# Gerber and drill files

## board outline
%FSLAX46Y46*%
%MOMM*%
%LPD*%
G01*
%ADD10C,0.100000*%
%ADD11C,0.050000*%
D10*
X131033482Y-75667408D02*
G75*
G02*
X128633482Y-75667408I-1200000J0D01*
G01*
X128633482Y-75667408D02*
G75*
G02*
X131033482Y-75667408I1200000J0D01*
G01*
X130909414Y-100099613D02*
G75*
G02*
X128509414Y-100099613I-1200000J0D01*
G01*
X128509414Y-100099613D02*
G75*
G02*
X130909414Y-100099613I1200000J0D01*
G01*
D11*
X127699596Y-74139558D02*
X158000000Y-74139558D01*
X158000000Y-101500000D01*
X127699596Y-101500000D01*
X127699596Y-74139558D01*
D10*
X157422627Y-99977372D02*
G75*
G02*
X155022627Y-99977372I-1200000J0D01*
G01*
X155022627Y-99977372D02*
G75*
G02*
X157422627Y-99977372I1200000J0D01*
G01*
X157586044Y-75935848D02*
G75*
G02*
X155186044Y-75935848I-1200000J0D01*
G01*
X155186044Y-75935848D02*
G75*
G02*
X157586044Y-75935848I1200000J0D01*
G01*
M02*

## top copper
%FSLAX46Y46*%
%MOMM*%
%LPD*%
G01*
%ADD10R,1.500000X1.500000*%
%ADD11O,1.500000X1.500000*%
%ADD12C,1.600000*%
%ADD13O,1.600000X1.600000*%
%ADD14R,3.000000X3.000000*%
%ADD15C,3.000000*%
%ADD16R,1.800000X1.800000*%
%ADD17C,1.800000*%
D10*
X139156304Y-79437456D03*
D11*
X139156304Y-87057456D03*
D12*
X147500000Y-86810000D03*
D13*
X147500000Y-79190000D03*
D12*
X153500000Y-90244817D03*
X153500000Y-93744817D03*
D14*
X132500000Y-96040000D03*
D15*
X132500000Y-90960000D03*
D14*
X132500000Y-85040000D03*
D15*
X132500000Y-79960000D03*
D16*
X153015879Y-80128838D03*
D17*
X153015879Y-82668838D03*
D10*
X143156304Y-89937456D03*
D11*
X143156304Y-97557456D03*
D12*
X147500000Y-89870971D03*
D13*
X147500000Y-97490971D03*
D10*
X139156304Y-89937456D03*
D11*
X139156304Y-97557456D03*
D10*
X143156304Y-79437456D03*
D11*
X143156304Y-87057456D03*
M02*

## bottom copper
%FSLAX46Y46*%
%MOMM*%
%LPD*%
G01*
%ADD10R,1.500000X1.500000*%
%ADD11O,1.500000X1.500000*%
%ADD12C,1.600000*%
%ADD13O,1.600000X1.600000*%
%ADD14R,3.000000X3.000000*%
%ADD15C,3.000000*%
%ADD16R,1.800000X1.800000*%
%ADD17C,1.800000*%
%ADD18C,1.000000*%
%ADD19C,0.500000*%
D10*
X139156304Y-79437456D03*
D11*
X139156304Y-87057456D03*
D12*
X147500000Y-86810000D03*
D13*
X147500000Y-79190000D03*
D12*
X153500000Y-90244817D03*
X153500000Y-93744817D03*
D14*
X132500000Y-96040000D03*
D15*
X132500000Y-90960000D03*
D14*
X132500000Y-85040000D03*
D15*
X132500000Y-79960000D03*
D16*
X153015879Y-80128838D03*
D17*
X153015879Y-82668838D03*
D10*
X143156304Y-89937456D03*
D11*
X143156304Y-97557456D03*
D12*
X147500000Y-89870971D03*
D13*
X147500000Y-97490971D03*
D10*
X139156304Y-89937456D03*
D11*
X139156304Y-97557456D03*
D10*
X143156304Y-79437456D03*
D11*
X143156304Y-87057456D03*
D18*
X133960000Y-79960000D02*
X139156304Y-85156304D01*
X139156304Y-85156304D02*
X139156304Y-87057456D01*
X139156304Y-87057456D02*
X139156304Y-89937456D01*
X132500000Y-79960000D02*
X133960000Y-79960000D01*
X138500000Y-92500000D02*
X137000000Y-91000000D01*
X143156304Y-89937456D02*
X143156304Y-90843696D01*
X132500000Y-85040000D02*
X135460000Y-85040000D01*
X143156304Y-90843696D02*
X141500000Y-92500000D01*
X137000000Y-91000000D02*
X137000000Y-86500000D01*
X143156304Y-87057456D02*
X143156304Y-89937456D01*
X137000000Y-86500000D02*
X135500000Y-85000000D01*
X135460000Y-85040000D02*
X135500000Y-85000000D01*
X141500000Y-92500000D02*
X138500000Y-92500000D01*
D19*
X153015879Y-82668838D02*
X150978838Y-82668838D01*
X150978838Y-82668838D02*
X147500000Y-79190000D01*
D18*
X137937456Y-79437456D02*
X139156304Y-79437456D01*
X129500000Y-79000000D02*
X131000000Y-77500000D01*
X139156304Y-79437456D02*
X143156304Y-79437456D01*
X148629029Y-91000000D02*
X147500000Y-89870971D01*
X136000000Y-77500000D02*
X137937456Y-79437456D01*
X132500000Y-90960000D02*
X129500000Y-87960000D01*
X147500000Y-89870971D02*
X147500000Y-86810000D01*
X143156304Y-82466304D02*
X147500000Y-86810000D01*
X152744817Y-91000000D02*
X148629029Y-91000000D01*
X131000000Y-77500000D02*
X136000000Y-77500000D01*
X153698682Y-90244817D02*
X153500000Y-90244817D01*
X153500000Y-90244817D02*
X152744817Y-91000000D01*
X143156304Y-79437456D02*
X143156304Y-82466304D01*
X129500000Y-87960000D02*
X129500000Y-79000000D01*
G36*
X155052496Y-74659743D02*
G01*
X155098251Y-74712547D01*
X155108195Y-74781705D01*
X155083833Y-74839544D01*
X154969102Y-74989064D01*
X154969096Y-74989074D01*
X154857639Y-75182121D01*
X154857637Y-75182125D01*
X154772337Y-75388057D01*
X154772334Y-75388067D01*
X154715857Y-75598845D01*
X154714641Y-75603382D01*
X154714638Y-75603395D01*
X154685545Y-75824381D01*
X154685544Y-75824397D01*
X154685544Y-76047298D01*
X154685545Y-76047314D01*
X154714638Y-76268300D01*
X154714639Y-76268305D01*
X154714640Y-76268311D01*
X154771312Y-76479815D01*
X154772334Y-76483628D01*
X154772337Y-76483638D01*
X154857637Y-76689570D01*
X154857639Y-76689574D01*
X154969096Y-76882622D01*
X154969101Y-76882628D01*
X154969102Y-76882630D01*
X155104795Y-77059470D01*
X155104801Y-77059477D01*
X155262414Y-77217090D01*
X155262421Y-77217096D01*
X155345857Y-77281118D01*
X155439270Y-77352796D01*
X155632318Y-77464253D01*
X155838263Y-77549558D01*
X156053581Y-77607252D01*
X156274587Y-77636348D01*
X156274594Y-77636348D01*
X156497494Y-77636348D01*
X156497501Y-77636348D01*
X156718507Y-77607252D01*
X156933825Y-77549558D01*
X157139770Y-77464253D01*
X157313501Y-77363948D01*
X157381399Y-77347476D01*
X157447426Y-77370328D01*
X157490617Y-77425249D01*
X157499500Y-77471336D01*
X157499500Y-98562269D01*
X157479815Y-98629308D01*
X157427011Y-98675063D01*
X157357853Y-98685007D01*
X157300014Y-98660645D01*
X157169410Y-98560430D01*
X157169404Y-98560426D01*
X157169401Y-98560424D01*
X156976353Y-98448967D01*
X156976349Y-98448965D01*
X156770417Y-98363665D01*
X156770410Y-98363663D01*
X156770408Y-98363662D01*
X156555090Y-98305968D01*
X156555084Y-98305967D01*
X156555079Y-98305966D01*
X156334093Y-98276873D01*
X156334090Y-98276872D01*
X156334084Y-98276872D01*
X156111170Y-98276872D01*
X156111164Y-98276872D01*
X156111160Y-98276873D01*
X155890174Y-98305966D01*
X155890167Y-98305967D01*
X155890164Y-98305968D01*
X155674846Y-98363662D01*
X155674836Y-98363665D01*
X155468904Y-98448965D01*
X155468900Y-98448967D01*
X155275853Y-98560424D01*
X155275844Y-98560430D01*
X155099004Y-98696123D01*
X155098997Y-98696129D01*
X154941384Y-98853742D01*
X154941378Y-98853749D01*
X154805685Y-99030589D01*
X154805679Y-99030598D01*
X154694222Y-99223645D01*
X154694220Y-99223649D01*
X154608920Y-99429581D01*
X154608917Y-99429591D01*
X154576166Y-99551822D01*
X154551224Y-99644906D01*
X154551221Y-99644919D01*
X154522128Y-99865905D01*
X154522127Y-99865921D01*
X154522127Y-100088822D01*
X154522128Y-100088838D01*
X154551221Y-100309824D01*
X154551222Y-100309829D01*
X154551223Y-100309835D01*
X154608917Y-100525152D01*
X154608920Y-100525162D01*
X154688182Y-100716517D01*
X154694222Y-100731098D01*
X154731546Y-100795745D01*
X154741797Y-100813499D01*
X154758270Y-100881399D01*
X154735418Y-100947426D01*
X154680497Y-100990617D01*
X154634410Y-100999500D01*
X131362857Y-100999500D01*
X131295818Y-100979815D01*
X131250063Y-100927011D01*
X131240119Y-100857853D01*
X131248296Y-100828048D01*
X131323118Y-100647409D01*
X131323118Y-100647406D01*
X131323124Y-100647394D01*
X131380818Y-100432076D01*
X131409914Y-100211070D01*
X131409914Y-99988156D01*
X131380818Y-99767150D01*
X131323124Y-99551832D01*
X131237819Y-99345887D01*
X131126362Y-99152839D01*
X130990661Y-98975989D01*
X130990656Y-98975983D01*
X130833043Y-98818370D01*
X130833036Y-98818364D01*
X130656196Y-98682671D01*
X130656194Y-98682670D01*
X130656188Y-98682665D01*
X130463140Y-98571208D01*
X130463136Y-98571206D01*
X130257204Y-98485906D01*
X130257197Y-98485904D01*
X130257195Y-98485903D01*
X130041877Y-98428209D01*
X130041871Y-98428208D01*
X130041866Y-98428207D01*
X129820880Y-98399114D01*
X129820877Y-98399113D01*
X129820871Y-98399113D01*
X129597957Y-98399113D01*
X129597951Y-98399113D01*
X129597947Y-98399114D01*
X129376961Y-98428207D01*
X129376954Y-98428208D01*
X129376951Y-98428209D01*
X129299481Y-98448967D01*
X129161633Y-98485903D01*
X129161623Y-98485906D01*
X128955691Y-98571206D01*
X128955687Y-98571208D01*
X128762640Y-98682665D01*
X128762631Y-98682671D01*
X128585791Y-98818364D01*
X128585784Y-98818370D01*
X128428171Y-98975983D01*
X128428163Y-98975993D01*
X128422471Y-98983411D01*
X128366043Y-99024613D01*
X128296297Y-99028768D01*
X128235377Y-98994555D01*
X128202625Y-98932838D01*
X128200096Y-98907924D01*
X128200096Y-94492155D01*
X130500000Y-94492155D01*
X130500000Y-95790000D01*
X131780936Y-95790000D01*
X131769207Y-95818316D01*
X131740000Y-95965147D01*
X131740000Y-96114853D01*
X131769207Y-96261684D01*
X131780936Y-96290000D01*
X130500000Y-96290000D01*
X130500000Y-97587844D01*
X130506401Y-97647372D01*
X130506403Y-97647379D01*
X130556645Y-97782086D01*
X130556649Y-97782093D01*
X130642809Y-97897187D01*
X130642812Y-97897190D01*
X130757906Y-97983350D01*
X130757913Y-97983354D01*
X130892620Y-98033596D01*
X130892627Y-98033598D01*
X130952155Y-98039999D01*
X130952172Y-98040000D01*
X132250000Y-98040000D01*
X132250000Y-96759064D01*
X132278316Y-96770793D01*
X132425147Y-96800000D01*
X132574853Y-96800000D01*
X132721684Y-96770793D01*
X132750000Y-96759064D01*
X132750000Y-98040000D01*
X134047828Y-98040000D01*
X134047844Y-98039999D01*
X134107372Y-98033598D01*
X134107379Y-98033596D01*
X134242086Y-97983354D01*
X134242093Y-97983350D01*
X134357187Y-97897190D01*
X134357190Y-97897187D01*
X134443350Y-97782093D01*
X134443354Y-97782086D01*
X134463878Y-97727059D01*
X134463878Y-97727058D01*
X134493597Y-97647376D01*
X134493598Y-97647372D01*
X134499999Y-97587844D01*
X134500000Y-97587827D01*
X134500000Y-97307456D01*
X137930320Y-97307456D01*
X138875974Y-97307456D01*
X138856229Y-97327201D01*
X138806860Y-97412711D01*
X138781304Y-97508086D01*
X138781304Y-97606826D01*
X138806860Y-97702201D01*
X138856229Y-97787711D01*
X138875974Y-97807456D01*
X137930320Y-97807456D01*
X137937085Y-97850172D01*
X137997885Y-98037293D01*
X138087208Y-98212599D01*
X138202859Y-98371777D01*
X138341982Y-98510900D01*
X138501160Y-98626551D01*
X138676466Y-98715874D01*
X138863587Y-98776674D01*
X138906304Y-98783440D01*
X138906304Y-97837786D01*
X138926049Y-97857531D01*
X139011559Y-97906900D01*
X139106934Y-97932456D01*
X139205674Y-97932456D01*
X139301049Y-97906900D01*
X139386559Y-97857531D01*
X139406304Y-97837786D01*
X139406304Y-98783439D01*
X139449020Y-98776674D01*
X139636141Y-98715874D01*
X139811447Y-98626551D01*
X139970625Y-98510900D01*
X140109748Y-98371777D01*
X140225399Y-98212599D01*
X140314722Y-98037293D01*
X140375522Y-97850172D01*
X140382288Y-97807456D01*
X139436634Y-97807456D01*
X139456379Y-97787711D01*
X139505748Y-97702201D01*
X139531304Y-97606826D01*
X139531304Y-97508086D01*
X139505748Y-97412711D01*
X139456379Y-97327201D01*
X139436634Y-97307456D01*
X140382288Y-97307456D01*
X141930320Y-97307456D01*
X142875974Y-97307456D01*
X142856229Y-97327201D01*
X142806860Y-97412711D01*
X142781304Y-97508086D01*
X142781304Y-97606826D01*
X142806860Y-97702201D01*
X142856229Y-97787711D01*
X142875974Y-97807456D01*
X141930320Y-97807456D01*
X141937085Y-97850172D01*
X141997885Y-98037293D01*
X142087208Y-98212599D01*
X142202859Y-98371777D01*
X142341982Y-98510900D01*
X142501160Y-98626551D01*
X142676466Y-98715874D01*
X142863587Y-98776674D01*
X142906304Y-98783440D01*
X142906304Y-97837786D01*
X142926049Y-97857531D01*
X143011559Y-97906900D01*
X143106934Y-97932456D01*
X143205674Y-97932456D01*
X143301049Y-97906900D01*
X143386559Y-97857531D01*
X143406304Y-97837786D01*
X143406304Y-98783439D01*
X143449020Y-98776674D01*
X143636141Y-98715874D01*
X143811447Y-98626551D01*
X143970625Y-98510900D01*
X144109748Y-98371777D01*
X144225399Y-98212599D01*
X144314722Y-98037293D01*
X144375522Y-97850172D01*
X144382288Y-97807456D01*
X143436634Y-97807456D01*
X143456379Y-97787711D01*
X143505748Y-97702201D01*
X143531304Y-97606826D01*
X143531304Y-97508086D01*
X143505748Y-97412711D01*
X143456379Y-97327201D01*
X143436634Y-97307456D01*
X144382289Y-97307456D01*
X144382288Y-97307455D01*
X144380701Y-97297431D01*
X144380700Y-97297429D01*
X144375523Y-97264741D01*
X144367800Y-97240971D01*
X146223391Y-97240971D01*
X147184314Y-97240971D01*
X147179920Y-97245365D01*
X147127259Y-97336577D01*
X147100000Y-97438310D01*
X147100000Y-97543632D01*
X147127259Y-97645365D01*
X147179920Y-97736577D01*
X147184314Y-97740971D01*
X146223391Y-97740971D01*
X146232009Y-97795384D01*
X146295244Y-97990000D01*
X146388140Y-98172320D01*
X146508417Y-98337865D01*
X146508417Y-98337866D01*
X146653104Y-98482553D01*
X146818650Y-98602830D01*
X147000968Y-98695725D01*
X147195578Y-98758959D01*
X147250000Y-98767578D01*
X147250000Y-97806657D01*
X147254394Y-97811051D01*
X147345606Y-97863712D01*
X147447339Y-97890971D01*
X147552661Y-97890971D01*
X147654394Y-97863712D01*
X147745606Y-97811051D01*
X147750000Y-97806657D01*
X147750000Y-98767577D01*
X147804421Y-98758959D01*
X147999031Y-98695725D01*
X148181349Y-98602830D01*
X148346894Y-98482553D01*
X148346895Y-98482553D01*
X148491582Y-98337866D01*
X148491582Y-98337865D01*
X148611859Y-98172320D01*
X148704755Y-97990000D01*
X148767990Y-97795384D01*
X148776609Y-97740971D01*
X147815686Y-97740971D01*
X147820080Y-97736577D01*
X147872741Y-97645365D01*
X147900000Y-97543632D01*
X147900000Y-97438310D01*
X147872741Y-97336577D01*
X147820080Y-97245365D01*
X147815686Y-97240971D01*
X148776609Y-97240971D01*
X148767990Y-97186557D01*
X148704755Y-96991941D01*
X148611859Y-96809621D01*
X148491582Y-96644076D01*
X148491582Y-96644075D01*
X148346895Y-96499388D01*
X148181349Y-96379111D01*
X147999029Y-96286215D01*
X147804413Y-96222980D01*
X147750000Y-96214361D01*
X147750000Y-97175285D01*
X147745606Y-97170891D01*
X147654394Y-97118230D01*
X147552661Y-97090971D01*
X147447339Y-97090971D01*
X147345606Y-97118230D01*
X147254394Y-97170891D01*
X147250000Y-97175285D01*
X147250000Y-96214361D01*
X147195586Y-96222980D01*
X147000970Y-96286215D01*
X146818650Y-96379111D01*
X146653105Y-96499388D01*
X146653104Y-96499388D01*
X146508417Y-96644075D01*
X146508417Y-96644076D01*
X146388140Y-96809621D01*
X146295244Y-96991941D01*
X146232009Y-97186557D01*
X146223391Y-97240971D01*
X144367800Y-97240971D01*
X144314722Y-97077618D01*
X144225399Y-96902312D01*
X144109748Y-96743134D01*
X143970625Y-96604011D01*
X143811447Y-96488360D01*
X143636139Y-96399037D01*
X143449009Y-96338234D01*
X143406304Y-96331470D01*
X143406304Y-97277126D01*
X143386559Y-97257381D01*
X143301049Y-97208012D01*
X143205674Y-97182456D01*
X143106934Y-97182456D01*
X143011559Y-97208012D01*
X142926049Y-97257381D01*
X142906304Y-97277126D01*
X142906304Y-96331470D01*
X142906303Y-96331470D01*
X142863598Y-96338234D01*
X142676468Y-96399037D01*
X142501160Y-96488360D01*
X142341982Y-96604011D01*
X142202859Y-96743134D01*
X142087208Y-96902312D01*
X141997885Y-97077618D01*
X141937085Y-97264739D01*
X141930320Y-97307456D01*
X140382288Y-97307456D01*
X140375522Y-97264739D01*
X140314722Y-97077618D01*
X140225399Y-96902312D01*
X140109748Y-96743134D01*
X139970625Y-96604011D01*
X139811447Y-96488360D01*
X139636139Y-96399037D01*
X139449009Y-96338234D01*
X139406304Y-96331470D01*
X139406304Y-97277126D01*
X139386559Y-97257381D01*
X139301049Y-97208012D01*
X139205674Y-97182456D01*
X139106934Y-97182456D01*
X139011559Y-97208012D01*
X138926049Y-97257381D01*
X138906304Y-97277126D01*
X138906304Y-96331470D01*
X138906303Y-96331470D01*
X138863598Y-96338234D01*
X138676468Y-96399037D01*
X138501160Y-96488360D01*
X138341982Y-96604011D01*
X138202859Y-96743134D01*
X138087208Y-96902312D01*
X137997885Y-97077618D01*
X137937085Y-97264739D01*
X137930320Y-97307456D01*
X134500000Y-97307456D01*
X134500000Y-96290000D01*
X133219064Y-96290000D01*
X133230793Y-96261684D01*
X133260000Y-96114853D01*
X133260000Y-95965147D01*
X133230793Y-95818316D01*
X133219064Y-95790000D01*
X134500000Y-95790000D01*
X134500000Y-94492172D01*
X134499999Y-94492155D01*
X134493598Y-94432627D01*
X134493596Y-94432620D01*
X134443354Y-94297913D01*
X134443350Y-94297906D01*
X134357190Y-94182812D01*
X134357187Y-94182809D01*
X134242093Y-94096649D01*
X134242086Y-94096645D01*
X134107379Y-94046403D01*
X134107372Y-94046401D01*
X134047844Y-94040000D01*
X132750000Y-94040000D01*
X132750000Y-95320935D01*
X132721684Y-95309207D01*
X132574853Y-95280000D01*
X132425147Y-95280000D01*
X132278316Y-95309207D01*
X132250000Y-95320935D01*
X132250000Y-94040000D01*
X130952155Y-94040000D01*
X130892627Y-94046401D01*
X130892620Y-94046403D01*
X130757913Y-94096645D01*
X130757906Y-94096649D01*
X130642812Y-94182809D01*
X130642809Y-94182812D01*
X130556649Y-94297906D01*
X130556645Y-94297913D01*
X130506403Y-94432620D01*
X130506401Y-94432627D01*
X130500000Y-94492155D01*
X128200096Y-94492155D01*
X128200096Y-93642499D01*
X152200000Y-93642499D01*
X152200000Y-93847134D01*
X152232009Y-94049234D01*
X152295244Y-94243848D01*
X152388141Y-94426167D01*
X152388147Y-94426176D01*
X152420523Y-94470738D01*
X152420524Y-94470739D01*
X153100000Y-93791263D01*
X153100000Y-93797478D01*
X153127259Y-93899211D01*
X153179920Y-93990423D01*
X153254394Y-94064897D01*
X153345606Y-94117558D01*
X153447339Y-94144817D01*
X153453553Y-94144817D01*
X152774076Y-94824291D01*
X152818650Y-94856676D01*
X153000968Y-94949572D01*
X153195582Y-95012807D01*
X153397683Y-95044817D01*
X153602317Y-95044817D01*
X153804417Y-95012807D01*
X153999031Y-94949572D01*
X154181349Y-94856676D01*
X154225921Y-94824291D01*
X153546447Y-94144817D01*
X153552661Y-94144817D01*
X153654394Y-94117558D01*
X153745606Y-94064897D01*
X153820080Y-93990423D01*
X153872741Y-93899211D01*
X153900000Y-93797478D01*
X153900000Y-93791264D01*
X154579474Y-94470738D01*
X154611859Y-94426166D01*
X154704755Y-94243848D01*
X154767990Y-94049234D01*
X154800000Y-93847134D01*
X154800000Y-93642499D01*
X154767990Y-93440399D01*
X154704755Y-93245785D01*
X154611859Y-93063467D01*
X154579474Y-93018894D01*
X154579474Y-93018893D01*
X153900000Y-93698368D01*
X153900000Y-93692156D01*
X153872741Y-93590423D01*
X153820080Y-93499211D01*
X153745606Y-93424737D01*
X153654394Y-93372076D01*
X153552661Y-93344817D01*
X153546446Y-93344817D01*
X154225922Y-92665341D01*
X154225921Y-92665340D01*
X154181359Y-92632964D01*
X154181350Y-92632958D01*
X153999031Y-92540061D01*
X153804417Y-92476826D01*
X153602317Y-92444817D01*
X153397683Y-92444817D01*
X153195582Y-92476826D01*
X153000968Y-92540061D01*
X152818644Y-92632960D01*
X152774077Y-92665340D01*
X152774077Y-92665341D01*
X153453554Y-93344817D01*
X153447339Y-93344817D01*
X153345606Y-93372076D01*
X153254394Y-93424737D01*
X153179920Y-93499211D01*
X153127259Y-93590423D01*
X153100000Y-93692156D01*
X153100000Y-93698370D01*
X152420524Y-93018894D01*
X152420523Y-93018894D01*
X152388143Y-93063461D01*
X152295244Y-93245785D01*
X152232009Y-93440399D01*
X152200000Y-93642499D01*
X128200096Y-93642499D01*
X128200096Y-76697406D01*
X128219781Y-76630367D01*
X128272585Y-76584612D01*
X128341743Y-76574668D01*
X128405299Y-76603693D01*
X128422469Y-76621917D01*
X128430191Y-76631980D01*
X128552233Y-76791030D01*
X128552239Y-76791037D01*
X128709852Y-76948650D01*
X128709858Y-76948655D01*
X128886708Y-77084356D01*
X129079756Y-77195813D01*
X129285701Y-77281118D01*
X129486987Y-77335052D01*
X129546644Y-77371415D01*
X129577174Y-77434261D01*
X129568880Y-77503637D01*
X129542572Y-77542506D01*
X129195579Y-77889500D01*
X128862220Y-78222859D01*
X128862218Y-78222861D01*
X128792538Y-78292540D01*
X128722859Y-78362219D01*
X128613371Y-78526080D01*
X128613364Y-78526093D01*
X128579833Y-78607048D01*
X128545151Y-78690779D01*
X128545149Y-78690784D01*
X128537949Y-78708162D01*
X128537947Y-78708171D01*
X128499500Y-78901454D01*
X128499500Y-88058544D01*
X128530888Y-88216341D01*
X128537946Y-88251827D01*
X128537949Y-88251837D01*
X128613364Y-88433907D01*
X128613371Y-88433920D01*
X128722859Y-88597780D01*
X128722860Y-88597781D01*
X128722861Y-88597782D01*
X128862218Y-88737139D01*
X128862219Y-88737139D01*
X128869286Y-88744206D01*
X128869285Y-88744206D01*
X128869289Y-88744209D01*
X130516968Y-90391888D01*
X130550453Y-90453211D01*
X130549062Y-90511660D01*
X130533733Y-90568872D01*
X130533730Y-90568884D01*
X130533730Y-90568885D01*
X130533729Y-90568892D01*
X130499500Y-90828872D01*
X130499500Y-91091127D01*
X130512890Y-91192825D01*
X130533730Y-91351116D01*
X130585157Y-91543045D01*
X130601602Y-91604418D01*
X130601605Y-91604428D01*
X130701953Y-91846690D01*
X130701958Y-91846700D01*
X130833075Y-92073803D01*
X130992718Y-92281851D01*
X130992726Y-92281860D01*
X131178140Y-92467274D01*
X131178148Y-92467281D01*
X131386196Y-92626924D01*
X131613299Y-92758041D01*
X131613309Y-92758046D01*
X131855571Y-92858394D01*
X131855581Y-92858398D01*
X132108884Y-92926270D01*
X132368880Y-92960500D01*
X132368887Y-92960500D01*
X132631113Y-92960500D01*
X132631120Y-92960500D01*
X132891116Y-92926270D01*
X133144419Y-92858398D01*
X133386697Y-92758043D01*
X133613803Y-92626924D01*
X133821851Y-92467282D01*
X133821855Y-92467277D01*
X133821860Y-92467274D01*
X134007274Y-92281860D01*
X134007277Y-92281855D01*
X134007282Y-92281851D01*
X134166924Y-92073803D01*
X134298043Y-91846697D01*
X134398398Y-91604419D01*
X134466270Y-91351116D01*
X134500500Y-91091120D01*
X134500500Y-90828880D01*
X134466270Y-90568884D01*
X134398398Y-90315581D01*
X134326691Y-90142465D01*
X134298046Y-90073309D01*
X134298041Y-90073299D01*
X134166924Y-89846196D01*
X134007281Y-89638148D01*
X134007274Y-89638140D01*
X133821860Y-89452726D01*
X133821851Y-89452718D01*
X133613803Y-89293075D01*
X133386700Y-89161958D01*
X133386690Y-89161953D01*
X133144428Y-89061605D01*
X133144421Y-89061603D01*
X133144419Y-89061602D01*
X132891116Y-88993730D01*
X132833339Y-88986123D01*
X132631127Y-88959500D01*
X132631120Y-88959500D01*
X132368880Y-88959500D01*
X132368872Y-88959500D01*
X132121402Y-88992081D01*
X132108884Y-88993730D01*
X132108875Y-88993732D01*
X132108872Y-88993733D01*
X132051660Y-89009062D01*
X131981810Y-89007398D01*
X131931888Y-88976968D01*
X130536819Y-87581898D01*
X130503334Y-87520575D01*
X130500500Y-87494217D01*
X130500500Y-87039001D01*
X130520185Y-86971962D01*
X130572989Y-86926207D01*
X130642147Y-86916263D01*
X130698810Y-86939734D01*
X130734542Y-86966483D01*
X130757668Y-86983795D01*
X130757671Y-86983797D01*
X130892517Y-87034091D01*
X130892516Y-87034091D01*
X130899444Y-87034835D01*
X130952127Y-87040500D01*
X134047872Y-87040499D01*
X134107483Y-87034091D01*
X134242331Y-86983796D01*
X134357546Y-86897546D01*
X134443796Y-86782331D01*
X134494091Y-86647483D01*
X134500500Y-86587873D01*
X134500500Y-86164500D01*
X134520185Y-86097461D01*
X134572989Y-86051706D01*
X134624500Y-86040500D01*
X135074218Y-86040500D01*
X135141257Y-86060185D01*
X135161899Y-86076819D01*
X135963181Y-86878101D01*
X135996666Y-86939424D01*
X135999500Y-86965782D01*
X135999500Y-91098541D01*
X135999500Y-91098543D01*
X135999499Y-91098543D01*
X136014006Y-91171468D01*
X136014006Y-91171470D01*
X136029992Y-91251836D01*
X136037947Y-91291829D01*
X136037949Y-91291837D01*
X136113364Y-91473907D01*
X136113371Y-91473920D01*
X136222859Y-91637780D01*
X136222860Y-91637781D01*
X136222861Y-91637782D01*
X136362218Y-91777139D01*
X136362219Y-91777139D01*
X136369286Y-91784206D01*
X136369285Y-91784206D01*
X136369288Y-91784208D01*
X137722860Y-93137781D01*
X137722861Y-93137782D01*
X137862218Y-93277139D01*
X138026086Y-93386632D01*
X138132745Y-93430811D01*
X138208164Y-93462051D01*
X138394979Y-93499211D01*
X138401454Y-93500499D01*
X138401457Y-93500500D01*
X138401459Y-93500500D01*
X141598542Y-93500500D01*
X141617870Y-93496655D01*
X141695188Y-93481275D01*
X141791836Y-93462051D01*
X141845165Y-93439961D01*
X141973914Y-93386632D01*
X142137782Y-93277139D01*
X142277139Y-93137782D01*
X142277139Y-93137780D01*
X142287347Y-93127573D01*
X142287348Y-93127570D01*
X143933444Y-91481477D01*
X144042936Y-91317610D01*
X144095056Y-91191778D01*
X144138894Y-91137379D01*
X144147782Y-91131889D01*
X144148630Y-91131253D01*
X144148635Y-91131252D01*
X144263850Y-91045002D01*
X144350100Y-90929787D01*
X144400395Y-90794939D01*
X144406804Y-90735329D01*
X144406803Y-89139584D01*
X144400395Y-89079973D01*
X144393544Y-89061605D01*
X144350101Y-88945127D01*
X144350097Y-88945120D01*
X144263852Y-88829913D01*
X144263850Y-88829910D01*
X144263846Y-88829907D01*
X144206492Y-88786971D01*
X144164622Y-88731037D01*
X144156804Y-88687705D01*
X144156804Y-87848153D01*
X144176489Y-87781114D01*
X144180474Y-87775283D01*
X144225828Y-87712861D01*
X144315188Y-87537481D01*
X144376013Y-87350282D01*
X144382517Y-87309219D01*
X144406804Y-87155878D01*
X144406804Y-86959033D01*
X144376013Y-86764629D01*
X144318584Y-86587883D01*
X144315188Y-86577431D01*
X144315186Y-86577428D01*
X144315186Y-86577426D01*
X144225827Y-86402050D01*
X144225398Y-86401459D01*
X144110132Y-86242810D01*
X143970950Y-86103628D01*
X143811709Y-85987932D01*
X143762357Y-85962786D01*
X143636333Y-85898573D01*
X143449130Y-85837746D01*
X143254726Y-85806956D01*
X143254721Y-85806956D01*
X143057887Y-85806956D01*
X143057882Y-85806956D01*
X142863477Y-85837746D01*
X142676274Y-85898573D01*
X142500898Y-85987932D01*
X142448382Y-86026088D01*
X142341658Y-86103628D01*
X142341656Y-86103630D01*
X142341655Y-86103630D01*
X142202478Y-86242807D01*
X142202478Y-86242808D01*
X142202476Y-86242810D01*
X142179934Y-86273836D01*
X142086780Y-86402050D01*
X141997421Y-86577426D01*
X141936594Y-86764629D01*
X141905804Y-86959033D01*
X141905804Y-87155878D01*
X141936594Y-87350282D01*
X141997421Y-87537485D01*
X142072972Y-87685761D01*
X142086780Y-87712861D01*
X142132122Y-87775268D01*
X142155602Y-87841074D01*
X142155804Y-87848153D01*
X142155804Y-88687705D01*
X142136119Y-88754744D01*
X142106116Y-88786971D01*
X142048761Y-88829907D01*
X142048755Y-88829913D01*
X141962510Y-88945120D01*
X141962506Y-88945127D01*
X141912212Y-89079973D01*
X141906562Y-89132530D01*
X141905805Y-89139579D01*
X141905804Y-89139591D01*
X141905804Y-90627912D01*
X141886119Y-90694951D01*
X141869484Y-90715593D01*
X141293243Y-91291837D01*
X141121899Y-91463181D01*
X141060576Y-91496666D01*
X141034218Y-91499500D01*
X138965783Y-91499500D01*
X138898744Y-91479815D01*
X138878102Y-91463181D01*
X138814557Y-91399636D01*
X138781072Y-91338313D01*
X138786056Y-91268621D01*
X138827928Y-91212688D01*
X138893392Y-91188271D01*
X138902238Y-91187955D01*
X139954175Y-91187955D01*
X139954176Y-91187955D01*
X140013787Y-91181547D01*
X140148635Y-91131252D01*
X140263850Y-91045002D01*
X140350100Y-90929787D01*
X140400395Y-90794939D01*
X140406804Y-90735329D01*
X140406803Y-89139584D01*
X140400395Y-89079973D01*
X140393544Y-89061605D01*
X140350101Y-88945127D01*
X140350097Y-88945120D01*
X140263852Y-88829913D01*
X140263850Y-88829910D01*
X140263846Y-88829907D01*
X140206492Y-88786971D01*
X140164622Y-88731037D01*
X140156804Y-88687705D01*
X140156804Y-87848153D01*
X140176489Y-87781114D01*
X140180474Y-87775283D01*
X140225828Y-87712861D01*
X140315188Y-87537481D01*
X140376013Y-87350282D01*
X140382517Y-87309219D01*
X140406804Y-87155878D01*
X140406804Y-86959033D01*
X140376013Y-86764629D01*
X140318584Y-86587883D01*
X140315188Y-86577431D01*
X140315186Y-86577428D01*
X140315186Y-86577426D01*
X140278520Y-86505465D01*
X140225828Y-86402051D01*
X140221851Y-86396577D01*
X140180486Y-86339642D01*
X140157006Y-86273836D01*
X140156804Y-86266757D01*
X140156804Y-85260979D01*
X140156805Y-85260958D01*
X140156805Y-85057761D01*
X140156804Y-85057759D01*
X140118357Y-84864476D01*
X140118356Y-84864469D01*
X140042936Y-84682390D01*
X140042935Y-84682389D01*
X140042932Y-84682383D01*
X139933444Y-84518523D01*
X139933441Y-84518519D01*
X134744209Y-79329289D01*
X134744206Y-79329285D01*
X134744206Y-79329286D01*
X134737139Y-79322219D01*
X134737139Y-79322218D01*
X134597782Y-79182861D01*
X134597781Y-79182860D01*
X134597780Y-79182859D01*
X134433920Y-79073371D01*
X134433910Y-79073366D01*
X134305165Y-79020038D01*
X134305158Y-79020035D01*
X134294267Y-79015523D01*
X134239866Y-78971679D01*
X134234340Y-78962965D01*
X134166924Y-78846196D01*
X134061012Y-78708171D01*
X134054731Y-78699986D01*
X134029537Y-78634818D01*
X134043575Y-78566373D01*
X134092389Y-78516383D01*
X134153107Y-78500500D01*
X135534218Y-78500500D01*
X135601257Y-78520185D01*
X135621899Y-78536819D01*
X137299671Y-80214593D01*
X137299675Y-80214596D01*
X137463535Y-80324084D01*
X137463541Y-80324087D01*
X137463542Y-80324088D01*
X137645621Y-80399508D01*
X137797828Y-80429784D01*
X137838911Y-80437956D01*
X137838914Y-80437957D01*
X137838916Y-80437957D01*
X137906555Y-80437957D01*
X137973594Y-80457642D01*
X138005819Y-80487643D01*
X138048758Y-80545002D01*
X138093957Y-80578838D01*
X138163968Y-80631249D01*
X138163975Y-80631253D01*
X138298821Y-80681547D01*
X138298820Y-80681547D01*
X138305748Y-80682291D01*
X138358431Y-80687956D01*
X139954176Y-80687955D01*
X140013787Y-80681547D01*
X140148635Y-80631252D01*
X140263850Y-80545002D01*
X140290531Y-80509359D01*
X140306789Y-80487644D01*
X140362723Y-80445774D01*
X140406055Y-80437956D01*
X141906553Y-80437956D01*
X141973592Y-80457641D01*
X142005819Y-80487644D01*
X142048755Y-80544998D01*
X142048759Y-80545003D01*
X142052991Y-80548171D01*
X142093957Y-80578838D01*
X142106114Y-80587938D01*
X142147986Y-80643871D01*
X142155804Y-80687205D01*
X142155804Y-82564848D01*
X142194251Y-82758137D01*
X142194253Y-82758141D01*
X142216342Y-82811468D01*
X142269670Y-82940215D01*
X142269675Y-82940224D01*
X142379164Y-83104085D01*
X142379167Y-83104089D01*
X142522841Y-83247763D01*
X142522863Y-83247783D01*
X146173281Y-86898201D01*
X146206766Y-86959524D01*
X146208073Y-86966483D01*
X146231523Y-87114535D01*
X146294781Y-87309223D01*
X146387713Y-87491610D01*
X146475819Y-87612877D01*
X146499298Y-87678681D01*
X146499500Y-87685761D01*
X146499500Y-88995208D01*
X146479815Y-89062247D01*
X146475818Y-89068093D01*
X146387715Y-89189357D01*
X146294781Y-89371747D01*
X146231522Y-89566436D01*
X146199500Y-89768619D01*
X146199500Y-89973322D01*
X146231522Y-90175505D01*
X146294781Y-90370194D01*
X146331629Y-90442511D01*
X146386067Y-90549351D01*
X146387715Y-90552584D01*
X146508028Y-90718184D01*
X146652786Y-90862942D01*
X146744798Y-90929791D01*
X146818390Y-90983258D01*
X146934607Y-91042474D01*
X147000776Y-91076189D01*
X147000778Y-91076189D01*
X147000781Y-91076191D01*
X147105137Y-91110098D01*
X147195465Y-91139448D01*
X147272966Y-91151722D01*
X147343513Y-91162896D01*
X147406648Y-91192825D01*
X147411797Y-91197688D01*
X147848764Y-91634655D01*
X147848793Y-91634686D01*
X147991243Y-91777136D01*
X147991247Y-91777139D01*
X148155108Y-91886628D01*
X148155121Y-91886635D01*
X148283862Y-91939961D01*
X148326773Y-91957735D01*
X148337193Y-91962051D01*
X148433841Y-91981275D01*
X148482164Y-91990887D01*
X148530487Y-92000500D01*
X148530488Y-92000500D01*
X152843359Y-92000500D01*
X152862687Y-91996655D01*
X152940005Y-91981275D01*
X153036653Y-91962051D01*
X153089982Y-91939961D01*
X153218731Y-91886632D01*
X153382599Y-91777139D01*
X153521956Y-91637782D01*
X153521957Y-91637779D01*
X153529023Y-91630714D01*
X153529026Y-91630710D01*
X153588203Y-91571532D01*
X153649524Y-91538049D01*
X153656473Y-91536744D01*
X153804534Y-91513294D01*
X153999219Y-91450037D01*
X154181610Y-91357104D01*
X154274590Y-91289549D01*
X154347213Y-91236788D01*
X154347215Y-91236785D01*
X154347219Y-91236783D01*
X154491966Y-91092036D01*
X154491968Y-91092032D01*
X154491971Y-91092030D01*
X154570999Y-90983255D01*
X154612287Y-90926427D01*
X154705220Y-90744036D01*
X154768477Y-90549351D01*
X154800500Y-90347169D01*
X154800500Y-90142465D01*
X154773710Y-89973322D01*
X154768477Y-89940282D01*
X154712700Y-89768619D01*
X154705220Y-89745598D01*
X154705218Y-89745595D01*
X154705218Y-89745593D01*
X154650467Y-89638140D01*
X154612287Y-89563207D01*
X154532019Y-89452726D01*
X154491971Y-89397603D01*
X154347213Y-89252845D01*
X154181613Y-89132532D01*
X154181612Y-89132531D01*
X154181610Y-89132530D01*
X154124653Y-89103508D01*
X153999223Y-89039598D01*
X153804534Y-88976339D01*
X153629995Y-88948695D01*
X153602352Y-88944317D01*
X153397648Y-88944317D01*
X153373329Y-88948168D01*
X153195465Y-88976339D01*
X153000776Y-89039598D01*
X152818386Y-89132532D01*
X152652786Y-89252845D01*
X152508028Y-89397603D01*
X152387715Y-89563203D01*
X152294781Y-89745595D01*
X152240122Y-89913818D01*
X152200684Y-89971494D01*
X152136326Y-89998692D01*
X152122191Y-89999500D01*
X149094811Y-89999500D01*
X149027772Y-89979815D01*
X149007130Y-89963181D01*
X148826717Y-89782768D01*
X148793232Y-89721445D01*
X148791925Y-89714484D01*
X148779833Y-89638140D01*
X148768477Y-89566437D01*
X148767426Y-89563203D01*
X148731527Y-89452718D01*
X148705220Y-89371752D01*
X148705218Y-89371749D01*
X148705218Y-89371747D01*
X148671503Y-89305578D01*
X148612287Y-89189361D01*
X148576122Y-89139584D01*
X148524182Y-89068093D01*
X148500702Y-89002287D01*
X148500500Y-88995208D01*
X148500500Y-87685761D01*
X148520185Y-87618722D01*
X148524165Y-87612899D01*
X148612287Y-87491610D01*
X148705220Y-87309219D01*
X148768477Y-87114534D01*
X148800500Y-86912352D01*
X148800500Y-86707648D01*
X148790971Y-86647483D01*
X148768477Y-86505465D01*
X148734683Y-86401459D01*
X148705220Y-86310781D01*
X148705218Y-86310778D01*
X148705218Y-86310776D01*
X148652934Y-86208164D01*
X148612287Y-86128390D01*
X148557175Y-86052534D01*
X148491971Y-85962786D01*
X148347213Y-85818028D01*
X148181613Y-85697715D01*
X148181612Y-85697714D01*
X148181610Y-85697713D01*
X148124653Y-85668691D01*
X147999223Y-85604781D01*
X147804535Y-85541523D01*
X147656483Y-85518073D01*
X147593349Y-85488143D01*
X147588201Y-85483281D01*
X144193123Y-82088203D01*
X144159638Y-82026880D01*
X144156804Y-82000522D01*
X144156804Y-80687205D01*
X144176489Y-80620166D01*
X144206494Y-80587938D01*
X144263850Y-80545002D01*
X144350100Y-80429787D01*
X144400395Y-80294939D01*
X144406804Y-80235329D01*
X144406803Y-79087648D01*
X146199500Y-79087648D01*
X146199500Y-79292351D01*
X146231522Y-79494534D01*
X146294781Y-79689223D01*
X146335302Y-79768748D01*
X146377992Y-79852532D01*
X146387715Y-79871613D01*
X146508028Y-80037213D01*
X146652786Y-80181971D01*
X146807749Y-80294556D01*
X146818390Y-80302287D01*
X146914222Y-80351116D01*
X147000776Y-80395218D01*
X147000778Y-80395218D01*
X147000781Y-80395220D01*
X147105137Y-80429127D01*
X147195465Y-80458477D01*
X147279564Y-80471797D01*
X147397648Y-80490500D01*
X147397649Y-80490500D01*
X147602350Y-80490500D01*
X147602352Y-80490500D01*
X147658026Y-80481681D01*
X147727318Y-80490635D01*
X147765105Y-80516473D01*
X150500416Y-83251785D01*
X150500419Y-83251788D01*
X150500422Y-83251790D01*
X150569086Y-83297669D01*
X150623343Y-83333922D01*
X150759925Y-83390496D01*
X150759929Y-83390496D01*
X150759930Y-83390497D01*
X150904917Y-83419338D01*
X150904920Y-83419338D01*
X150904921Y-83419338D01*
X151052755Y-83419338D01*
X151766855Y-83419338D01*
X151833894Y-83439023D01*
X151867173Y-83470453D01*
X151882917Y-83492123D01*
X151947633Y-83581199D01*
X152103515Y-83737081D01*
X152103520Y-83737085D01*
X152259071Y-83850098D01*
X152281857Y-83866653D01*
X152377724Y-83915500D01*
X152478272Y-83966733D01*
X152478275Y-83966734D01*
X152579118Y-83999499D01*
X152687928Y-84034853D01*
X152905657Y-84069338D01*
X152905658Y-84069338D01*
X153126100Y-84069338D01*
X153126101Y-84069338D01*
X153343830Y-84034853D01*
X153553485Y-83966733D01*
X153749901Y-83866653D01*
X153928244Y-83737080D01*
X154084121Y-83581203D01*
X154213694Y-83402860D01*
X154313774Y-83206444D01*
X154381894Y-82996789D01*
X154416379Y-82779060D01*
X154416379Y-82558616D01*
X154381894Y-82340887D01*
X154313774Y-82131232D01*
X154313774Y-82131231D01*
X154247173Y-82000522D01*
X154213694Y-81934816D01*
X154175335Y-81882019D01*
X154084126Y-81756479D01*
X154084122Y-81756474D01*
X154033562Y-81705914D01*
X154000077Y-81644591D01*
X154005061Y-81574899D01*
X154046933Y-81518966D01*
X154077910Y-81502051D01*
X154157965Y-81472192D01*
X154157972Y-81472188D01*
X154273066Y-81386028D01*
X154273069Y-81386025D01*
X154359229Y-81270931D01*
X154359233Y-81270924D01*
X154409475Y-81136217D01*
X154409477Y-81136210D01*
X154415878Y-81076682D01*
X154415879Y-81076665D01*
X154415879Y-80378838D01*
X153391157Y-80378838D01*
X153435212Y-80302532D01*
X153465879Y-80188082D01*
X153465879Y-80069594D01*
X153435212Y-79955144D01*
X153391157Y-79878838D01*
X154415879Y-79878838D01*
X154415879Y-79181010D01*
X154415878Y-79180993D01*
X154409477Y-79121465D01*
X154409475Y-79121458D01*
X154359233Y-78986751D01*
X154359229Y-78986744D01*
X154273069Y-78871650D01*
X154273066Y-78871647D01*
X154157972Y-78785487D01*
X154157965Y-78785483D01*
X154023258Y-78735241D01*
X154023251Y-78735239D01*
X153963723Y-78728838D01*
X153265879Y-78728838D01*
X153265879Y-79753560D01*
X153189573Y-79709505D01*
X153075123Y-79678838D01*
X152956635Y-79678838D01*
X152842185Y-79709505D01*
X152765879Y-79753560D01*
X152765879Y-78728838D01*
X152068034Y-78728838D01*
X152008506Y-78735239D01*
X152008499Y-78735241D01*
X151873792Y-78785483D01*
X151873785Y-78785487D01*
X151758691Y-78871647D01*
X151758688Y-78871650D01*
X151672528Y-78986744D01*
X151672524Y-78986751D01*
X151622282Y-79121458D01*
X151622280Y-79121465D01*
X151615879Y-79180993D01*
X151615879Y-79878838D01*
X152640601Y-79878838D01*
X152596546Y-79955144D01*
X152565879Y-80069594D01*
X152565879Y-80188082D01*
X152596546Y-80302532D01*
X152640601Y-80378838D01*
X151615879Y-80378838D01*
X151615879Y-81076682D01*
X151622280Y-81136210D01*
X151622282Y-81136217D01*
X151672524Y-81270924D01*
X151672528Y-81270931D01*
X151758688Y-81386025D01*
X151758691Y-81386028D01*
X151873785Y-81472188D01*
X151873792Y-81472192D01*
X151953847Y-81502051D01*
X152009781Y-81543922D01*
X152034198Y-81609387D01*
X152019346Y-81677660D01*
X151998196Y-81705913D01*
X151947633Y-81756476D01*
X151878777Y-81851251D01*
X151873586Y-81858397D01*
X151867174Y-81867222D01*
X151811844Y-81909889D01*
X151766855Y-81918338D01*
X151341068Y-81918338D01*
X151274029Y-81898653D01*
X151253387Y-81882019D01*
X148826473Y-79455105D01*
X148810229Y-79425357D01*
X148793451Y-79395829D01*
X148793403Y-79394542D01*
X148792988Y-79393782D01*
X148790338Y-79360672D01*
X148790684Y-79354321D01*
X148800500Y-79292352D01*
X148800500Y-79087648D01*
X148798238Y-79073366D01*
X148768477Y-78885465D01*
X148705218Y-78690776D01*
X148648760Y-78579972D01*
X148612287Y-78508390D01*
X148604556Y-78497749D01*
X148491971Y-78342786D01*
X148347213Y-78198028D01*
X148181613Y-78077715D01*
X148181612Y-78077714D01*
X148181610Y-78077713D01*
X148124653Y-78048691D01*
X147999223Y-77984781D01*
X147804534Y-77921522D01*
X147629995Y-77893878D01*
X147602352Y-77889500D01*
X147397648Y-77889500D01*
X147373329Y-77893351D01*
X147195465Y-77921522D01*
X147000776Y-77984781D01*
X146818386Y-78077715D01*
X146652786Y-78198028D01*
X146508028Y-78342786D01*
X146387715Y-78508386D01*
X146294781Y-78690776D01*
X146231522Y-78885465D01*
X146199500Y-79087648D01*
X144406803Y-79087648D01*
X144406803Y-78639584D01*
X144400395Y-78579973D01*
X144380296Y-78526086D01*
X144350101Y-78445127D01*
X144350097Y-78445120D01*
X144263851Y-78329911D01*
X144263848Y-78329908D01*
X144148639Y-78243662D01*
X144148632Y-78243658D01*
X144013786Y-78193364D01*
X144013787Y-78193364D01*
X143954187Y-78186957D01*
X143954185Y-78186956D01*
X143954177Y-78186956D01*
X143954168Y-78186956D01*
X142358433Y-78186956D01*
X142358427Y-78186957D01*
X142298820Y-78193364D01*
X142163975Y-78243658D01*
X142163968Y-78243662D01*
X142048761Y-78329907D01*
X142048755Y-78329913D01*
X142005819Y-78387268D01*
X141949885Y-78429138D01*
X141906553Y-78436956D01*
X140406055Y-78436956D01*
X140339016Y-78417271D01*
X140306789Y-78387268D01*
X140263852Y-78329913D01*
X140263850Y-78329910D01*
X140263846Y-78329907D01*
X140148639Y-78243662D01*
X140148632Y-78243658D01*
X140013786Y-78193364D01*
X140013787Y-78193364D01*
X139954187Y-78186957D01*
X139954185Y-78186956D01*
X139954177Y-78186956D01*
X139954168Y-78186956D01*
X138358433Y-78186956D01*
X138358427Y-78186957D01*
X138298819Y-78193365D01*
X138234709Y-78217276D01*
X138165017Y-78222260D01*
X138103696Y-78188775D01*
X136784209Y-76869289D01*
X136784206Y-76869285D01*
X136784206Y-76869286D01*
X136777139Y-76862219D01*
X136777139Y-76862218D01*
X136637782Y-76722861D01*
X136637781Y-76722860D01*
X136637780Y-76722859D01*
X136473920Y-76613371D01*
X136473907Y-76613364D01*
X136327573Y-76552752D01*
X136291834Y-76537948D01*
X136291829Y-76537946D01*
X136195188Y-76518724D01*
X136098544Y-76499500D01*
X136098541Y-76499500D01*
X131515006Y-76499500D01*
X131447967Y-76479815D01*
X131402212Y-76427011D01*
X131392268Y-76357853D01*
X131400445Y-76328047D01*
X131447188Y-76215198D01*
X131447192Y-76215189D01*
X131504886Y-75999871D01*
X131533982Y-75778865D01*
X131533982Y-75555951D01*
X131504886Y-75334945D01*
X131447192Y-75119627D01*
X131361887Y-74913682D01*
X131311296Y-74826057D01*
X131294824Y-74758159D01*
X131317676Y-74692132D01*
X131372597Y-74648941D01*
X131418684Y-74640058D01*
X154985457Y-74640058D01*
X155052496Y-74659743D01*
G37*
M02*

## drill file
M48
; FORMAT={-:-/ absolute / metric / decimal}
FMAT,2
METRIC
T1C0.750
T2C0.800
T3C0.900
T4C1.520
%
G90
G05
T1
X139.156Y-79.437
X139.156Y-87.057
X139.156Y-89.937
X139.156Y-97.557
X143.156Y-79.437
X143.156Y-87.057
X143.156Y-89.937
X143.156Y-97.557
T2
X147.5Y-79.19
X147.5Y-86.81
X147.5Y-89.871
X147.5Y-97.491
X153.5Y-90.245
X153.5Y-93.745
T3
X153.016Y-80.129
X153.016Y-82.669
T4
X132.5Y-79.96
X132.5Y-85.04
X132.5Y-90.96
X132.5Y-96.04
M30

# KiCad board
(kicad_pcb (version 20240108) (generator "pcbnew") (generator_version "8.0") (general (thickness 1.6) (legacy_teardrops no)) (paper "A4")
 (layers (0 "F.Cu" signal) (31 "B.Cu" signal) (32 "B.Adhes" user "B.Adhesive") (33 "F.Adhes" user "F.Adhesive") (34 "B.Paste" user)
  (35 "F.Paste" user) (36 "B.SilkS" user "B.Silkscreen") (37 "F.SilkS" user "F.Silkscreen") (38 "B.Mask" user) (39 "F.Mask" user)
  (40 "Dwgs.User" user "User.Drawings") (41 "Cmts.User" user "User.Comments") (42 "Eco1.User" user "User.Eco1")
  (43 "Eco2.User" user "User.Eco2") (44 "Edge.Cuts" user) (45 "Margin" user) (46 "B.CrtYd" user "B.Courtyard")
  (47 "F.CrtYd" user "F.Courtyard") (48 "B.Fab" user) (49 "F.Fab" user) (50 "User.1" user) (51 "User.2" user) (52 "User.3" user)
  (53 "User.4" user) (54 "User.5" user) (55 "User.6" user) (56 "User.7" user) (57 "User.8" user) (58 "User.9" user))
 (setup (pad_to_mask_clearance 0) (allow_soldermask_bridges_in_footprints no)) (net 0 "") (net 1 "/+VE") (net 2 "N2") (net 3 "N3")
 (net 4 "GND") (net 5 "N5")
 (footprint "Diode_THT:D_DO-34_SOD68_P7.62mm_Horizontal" (layer "F.Cu") (at 139.156304 79.437456 -90)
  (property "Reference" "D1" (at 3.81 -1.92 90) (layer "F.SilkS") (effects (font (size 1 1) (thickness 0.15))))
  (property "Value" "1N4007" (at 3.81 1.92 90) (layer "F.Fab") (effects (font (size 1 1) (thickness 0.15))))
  (pad "1" thru_hole rect (at 0 0 270) (size 1.5 1.5) (drill 0.75) (layers "*.Cu" "*.Mask") (remove_unused_layers no) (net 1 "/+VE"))
  (pad "2" thru_hole oval (at 7.62 0 270) (size 1.5 1.5) (drill 0.75) (layers "*.Cu" "*.Mask") (remove_unused_layers no) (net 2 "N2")))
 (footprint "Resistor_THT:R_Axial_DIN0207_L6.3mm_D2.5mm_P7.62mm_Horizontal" (layer "F.Cu") (at 147.5 86.81 90)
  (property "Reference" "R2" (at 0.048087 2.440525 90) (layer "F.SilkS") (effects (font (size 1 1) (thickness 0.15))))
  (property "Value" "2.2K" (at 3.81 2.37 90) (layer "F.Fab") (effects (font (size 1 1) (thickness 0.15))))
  (pad "1" thru_hole circle (at 0 0 90) (size 1.6 1.6) (drill 0.8) (layers "*.Cu" "*.Mask") (remove_unused_layers no) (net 1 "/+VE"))
  (pad "2" thru_hole oval (at 7.62 0 90) (size 1.6 1.6) (drill 0.8) (layers "*.Cu" "*.Mask") (remove_unused_layers no) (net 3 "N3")))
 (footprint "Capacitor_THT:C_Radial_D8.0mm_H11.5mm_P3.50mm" (layer "F.Cu") (at 153.5 90.244817 -90)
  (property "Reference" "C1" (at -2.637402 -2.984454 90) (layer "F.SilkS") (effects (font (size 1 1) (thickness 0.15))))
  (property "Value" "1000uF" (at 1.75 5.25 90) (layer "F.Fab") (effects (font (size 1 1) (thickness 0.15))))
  (pad "1" thru_hole circle (at 0 0 270) (size 1.6 1.6) (drill 0.8) (layers "*.Cu" "*.Mask") (remove_unused_layers no) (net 1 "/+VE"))
  (pad "2" thru_hole circle (at 3.5 0 270) (size 1.6 1.6) (drill 0.8) (layers "*.Cu" "*.Mask") (remove_unused_layers no) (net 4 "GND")))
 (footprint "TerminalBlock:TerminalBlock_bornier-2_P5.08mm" (layer "F.Cu") (at 132.5 96.04 90)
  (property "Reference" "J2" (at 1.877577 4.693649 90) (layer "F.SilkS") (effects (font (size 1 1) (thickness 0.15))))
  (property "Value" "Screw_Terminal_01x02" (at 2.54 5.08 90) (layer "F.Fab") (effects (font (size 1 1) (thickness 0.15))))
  (pad "1" thru_hole rect (at 0 0 90) (size 3 3) (drill 1.52) (layers "*.Cu" "*.Mask") (remove_unused_layers no) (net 4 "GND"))
  (pad "2" thru_hole circle (at 5.08 0 90) (size 3 3) (drill 1.52) (layers "*.Cu" "*.Mask") (remove_unused_layers no) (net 1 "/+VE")))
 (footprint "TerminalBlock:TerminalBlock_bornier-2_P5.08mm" (layer "F.Cu") (at 132.5 85.04 90)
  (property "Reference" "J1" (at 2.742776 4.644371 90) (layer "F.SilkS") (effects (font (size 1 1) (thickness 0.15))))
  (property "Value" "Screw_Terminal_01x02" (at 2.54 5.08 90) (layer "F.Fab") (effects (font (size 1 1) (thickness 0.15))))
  (pad "1" thru_hole rect (at 0 0 90) (size 3 3) (drill 1.52) (layers "*.Cu" "*.Mask") (remove_unused_layers no) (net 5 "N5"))
  (pad "2" thru_hole circle (at 5.08 0 90) (size 3 3) (drill 1.52) (layers "*.Cu" "*.Mask") (remove_unused_layers no) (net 2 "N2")))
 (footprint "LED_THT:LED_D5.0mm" (layer "F.Cu") (at 153.015879 80.128838 -90)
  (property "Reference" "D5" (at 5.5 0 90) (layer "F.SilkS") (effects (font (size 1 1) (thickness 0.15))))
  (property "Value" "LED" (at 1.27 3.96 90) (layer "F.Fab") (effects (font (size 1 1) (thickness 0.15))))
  (pad "1" thru_hole rect (at 0 0 270) (size 1.8 1.8) (drill 0.9) (layers "*.Cu" "*.Mask") (remove_unused_layers no) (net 4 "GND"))
  (pad "2" thru_hole circle (at 2.54 0 270) (size 1.8 1.8) (drill 0.9) (layers "*.Cu" "*.Mask") (remove_unused_layers no) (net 3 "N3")))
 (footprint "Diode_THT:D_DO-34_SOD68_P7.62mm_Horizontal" (layer "F.Cu") (at 143.156304 89.937456 -90)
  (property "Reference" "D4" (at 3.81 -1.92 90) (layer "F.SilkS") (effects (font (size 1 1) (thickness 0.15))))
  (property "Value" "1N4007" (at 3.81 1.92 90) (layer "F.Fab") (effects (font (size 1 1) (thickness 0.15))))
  (pad "1" thru_hole rect (at 0 0 270) (size 1.5 1.5) (drill 0.75) (layers "*.Cu" "*.Mask") (remove_unused_layers no) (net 5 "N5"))
  (pad "2" thru_hole oval (at 7.62 0 270) (size 1.5 1.5) (drill 0.75) (layers "*.Cu" "*.Mask") (remove_unused_layers no) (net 4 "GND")))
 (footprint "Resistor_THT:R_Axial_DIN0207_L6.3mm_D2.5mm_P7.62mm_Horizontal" (layer "F.Cu") (at 147.5 89.870971 -90)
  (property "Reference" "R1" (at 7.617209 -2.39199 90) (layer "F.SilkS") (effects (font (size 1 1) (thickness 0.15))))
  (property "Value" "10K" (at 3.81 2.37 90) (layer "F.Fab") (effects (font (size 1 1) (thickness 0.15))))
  (pad "1" thru_hole circle (at 0 0 270) (size 1.6 1.6) (drill 0.8) (layers "*.Cu" "*.Mask") (remove_unused_layers no) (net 1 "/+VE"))
  (pad "2" thru_hole oval (at 7.62 0 270) (size 1.6 1.6) (drill 0.8) (layers "*.Cu" "*.Mask") (remove_unused_layers no) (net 4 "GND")))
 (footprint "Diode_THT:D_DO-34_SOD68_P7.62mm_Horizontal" (layer "F.Cu") (at 139.156304 89.937456 -90)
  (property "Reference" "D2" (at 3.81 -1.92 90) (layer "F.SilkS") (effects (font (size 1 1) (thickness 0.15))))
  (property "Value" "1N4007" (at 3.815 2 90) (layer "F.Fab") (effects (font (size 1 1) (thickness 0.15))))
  (pad "1" thru_hole rect (at 0 0 270) (size 1.5 1.5) (drill 0.75) (layers "*.Cu" "*.Mask") (remove_unused_layers no) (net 2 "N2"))
  (pad "2" thru_hole oval (at 7.62 0 270) (size 1.5 1.5) (drill 0.75) (layers "*.Cu" "*.Mask") (remove_unused_layers no) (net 4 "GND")))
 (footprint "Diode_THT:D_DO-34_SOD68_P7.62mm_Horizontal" (layer "F.Cu") (at 143.156304 79.437456 -90)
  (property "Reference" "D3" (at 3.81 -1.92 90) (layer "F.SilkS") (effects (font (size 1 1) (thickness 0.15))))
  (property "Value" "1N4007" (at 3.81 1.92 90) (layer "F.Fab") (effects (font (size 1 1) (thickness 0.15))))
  (pad "1" thru_hole rect (at 0 0 270) (size 1.5 1.5) (drill 0.75) (layers "*.Cu" "*.Mask") (remove_unused_layers no) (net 1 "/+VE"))
  (pad "2" thru_hole oval (at 7.62 0 270) (size 1.5 1.5) (drill 0.75) (layers "*.Cu" "*.Mask") (remove_unused_layers no) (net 5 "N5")))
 (gr_circle (center 129.833482 75.667408) (end 131.033482 75.667408) (stroke (width 0.1) (type default)) (fill none) (layer "Edge.Cuts"))
 (gr_circle (center 129.709414 100.099613) (end 130.909414 100.099613) (stroke (width 0.1) (type default)) (fill none) (layer "Edge.Cuts"))
 (gr_rect (start 127.699596 74.139558) (end 158 101.5) (stroke (width 0.05) (type default)) (fill none) (layer "Edge.Cuts"))
 (gr_circle (center 156.222627 99.977372) (end 157.422627 99.977372) (stroke (width 0.1) (type default)) (fill none) (layer "Edge.Cuts"))
 (gr_circle (center 156.386044 75.935848) (end 157.586044 75.935848) (stroke (width 0.1) (type default)) (fill none) (layer "Edge.Cuts"))
 (segment (start 133.96 79.96) (end 139.156304 85.156304) (width 1) (layer "B.Cu") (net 2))
 (segment (start 139.156304 85.156304) (end 139.156304 87.057456) (width 1) (layer "B.Cu") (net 2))
 (segment (start 139.156304 87.057456) (end 139.156304 89.937456) (width 1) (layer "B.Cu") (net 2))
 (segment (start 132.5 79.96) (end 133.96 79.96) (width 1) (layer "B.Cu") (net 2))
 (segment (start 138.5 92.5) (end 137 91) (width 1) (layer "B.Cu") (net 5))
 (segment (start 143.156304 89.937456) (end 143.156304 90.843696) (width 1) (layer "B.Cu") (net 5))
 (segment (start 132.5 85.04) (end 135.46 85.04) (width 1) (layer "B.Cu") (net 5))
 (segment (start 143.156304 90.843696) (end 141.5 92.5) (width 1) (layer "B.Cu") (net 5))
 (segment (start 137 91) (end 137 86.5) (width 1) (layer "B.Cu") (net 5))
 (segment (start 143.156304 87.057456) (end 143.156304 89.937456) (width 1) (layer "B.Cu") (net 5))
 (segment (start 137 86.5) (end 135.5 85) (width 1) (layer "B.Cu") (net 5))
 (segment (start 135.46 85.04) (end 135.5 85) (width 1) (layer "B.Cu") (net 5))
 (segment (start 141.5 92.5) (end 138.5 92.5) (width 1) (layer "B.Cu") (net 5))
 (segment (start 153.015879 82.668838) (end 150.978838 82.668838) (width 0.5) (layer "B.Cu") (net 3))
 (segment (start 150.978838 82.668838) (end 147.5 79.19) (width 0.5) (layer "B.Cu") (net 3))
 (segment (start 137.937456 79.437456) (end 139.156304 79.437456) (width 1) (layer "B.Cu") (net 1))
 (segment (start 129.5 79) (end 131 77.5) (width 1) (layer "B.Cu") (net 1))
 (segment (start 139.156304 79.437456) (end 143.156304 79.437456) (width 1) (layer "B.Cu") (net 1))
 (segment (start 148.629029 91) (end 147.5 89.870971) (width 1) (layer "B.Cu") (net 1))
 (segment (start 136 77.5) (end 137.937456 79.437456) (width 1) (layer "B.Cu") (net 1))
 (segment (start 132.5 90.96) (end 129.5 87.96) (width 1) (layer "B.Cu") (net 1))
 (segment (start 147.5 89.870971) (end 147.5 86.81) (width 1) (layer "B.Cu") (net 1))
 (segment (start 143.156304 82.466304) (end 147.5 86.81) (width 1) (layer "B.Cu") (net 1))
 (segment (start 152.744817 91) (end 148.629029 91) (width 1) (layer "B.Cu") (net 1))
 (segment (start 131 77.5) (end 136 77.5) (width 1) (layer "B.Cu") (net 1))
 (segment (start 153.698682 90.244817) (end 153.5 90.244817) (width 1) (layer "B.Cu") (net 1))
 (segment (start 153.5 90.244817) (end 152.744817 91) (width 1) (layer "B.Cu") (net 1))
 (segment (start 143.156304 79.437456) (end 143.156304 82.466304) (width 1) (layer "B.Cu") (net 1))
 (segment (start 129.5 87.96) (end 129.5 79) (width 1) (layer "B.Cu") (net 1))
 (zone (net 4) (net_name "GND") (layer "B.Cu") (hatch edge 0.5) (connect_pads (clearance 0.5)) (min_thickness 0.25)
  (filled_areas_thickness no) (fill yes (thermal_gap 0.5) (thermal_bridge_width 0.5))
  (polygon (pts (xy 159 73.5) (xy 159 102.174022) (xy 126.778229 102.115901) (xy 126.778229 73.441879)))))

